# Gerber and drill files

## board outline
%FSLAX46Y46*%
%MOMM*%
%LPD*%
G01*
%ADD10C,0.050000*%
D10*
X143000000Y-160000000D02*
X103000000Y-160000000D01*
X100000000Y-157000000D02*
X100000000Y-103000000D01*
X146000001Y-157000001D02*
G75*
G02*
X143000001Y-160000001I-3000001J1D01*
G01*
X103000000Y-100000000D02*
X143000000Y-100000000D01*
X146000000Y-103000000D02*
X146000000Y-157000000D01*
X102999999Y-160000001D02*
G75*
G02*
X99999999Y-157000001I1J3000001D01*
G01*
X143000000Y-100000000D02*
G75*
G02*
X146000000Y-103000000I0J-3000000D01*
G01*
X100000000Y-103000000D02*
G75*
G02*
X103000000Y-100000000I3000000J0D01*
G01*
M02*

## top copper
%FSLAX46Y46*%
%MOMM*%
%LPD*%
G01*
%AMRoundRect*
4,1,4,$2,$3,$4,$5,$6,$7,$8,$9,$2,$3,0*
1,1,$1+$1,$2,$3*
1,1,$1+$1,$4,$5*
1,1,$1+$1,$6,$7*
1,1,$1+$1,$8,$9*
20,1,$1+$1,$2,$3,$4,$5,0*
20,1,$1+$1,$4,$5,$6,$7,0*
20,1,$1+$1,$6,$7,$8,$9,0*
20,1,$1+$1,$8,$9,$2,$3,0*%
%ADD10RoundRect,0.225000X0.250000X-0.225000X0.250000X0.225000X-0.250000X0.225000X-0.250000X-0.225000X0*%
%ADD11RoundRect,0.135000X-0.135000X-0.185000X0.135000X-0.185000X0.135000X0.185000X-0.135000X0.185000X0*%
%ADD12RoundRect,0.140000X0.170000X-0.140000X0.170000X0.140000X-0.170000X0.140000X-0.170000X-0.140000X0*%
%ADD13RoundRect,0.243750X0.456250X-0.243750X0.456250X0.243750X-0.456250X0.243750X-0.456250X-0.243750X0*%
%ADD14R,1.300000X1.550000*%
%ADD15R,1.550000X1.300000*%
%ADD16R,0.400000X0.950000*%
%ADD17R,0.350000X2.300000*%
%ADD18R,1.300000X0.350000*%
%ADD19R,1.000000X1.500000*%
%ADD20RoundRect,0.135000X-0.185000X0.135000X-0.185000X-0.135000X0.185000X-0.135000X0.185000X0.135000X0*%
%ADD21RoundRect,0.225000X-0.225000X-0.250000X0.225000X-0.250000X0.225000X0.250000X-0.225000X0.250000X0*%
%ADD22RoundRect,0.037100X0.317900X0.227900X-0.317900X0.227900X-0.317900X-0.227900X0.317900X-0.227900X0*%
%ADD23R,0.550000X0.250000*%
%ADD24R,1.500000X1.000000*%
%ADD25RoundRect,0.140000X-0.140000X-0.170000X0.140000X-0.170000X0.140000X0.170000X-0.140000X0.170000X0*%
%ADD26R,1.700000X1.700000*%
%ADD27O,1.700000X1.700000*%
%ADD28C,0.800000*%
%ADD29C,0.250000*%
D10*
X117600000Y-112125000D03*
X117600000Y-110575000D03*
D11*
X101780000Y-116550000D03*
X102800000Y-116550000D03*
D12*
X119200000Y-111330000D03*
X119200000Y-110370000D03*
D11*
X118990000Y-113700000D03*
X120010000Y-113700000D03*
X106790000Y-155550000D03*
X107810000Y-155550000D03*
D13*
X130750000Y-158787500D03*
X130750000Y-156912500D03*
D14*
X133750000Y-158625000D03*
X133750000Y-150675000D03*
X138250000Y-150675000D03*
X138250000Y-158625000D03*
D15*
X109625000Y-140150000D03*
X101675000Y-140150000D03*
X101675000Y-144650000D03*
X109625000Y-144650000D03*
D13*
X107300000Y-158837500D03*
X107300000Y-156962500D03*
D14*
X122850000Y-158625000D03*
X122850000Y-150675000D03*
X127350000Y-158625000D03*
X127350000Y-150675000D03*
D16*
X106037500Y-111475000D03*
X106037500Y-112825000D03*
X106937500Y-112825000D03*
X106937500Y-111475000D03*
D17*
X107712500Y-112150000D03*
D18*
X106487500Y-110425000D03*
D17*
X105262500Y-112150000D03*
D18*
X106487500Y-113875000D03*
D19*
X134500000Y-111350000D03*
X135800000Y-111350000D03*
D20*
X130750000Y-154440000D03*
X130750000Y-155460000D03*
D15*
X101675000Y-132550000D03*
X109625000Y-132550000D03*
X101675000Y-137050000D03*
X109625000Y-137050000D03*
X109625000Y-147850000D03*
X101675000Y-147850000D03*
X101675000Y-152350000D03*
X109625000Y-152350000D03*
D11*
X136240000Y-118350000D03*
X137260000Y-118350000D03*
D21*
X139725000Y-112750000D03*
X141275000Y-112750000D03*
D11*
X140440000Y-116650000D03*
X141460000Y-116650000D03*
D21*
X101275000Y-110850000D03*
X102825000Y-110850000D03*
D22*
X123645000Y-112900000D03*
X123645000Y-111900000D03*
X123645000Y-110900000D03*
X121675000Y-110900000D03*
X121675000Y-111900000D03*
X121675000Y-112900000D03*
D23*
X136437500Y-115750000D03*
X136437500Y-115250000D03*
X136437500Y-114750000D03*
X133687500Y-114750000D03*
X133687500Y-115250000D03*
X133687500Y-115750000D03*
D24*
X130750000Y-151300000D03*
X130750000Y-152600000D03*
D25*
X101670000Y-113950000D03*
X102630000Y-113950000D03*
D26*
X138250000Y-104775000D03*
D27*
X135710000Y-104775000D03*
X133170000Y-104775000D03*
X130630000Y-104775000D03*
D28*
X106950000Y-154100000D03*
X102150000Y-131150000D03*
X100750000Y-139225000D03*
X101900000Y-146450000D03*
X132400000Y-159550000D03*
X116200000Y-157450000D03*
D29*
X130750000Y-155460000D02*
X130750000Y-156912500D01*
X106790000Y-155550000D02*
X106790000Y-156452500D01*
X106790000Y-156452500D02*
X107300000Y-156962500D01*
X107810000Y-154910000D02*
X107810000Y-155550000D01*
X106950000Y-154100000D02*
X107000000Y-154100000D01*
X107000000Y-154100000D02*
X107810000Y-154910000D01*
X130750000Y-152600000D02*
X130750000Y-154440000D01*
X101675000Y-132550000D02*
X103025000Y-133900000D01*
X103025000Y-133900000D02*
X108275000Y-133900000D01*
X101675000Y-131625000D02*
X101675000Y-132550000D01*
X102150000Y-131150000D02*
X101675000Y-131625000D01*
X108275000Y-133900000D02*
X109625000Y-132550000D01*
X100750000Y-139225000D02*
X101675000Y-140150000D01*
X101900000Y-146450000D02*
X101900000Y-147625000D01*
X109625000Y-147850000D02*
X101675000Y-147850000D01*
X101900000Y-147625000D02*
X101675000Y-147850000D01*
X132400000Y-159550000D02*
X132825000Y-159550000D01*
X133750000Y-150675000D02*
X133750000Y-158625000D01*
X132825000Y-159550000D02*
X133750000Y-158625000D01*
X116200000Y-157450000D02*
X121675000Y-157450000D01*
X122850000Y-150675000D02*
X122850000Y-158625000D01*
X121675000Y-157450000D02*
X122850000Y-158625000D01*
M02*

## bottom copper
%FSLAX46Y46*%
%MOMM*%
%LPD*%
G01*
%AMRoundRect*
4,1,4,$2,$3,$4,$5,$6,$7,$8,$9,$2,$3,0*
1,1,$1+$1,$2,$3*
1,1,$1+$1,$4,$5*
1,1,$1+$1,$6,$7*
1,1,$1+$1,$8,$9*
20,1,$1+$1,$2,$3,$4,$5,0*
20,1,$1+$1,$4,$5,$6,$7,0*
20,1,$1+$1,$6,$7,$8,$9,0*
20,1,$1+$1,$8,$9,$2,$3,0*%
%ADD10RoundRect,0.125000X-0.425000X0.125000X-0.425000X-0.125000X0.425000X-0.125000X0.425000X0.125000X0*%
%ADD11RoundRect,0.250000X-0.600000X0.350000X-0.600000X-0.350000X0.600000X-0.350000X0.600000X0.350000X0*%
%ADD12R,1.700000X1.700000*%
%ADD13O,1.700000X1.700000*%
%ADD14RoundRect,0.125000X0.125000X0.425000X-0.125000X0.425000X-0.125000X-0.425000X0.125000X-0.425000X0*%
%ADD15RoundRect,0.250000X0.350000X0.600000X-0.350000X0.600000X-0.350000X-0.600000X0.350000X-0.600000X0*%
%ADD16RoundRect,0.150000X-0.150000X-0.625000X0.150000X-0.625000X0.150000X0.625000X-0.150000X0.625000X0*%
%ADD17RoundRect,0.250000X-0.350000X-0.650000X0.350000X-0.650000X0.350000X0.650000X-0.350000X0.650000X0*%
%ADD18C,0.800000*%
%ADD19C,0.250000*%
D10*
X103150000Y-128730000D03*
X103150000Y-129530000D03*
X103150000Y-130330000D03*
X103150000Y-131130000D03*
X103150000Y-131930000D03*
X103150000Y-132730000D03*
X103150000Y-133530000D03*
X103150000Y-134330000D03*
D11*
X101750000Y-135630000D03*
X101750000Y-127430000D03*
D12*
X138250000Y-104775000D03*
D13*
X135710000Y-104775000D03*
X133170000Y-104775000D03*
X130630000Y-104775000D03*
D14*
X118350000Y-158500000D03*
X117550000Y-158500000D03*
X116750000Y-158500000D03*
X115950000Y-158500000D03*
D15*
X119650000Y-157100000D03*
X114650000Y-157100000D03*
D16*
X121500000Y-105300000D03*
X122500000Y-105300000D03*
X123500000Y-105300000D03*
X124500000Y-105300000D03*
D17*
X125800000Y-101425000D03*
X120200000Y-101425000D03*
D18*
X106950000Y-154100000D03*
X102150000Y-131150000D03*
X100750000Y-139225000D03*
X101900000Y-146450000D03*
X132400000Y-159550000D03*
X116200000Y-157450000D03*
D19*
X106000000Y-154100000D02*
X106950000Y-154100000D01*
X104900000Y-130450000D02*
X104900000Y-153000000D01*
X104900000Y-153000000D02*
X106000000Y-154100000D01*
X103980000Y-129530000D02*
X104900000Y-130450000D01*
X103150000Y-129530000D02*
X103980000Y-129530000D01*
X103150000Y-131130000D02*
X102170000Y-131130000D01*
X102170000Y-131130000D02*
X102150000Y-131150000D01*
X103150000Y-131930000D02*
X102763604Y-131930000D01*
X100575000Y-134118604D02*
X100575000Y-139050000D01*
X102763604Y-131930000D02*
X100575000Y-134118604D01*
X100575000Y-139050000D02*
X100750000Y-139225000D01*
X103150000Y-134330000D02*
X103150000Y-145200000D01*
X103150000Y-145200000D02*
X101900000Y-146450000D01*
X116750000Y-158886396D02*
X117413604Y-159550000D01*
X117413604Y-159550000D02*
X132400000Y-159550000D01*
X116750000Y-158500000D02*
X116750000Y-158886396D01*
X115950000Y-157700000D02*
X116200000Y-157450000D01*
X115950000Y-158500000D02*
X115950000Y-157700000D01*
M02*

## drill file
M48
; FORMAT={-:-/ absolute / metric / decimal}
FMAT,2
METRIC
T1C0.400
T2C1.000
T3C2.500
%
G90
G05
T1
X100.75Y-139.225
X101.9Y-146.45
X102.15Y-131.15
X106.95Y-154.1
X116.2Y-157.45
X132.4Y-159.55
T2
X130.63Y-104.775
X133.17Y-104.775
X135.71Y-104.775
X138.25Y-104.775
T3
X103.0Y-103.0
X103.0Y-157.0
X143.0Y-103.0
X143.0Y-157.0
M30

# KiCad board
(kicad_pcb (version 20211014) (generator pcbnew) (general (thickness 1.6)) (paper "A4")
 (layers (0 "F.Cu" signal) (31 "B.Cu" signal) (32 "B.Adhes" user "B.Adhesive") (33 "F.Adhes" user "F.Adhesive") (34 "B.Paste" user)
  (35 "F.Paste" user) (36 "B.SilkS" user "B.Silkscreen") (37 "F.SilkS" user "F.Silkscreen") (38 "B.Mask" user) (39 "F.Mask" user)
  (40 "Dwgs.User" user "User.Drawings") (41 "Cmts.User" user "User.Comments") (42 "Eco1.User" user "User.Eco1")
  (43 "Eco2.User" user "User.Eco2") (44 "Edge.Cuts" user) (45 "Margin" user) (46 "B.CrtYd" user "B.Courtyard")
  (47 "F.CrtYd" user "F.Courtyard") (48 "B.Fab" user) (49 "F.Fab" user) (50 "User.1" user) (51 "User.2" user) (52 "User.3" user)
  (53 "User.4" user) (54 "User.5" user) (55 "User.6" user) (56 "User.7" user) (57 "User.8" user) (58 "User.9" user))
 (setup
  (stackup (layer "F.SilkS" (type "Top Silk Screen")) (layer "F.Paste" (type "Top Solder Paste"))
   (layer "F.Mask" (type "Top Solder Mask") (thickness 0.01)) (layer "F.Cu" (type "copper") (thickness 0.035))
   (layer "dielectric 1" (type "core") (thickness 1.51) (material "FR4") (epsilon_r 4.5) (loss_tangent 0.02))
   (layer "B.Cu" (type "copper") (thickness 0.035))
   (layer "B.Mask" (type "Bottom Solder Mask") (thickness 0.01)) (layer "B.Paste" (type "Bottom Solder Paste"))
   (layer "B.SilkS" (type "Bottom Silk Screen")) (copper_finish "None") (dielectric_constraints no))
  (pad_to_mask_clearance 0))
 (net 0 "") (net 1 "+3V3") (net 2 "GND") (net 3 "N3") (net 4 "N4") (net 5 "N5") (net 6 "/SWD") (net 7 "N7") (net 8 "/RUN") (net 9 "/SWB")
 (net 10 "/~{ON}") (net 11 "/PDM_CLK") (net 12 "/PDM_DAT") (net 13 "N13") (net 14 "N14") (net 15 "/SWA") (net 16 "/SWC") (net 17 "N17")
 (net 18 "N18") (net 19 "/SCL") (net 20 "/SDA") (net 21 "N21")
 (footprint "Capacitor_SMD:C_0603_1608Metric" (layer "F.Cu") (at 117.6 111.35 90)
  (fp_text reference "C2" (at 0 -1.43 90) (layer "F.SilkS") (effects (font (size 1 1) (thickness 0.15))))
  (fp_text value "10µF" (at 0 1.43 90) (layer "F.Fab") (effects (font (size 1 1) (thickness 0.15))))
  (pad "1" smd roundrect (at -0.775 0 90) (size 0.9 0.95) (layers "F.Cu" "F.Paste" "F.Mask") (roundrect_rratio 0.25) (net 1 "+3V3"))
  (pad "2" smd roundrect (at 0.775 0 90) (size 0.9 0.95) (layers "F.Cu" "F.Paste" "F.Mask") (roundrect_rratio 0.25) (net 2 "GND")))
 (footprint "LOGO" (layer "F.Cu") (at 123.25 129.55)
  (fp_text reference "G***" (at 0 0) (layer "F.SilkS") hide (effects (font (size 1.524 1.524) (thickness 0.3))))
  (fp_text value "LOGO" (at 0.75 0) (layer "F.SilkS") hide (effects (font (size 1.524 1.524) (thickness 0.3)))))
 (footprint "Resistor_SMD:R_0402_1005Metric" (layer "F.Cu") (at 102.29 116.55)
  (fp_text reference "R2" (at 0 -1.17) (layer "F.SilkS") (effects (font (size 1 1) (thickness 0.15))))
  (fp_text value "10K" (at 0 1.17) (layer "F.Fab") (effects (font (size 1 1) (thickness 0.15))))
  (pad "1" smd roundrect (at -0.51 0) (size 0.54 0.64) (layers "F.Cu" "F.Paste" "F.Mask") (roundrect_rratio 0.25) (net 2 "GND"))
  (pad "2" smd roundrect (at 0.51 0) (size 0.54 0.64) (layers "F.Cu" "F.Paste" "F.Mask") (roundrect_rratio 0.25) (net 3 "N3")))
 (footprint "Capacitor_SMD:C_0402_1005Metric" (layer "F.Cu") (at 119.2 110.85 90)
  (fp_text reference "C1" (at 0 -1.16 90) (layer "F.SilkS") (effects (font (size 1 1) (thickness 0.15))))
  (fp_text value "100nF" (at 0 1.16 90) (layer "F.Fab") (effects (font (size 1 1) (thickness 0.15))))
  (pad "1" smd roundrect (at -0.48 0 90) (size 0.56 0.62) (layers "F.Cu" "F.Paste" "F.Mask") (roundrect_rratio 0.25) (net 1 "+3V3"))
  (pad "2" smd roundrect (at 0.48 0 90) (size 0.56 0.62) (layers "F.Cu" "F.Paste" "F.Mask") (roundrect_rratio 0.25) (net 2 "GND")))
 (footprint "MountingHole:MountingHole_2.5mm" (layer "F.Cu") (at 103 103)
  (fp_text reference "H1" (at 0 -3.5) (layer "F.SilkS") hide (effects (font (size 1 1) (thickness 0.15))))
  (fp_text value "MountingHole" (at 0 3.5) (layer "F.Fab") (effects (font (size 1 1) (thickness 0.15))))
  (pad "" np_thru_hole circle (at 0 0) (size 2.5 2.5) (drill 2.5) (layers *.Cu *.Mask)))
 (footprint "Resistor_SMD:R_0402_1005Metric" (layer "F.Cu") (at 119.5 113.7)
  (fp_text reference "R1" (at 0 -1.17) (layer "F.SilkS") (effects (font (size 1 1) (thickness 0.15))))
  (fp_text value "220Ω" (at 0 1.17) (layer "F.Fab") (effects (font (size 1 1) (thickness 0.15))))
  (pad "1" smd roundrect (at -0.51 0) (size 0.54 0.64) (layers "F.Cu" "F.Paste" "F.Mask") (roundrect_rratio 0.25) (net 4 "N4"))
  (pad "2" smd roundrect (at 0.51 0) (size 0.54 0.64) (layers "F.Cu" "F.Paste" "F.Mask") (roundrect_rratio 0.25) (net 1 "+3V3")))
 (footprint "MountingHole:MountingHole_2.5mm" (layer "F.Cu") (at 143 103)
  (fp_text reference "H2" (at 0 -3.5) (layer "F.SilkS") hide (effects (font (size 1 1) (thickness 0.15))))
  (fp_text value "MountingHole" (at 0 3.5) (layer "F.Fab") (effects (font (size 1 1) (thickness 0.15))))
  (pad "" np_thru_hole circle (at 0 0) (size 2.5 2.5) (drill 2.5) (layers *.Cu *.Mask)))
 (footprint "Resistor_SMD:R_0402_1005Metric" (layer "F.Cu") (at 107.3 155.55)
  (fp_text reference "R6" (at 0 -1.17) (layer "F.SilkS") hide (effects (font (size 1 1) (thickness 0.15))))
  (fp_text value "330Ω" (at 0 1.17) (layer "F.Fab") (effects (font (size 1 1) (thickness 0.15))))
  (pad "1" smd roundrect (at -0.51 0) (size 0.54 0.64) (layers "F.Cu" "F.Paste" "F.Mask") (roundrect_rratio 0.25) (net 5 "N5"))
  (pad "2" smd roundrect (at 0.51 0) (size 0.54 0.64) (layers "F.Cu" "F.Paste" "F.Mask") (roundrect_rratio 0.25) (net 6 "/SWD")))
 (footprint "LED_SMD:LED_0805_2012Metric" (layer "F.Cu") (at 130.75 157.85 90)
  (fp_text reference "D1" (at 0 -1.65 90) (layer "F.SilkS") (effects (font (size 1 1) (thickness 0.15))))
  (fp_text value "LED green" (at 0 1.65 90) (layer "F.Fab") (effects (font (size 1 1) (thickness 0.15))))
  (pad "1" smd roundrect (at -0.9375 0 90) (size 0.975 1.4) (layers "F.Cu" "F.Paste" "F.Mask") (roundrect_rratio 0.25) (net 2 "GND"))
  (pad "2" smd roundrect (at 0.9375 0 90) (size 0.975 1.4) (layers "F.Cu" "F.Paste" "F.Mask") (roundrect_rratio 0.25) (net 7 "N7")))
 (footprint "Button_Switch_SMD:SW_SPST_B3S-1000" (layer "F.Cu") (at 136 154.65 90)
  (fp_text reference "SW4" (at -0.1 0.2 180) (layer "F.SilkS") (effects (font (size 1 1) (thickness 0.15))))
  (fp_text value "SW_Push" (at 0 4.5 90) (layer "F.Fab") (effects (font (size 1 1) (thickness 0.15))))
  (pad "1" smd rect (at -3.975 -2.25 90) (size 1.55 1.3) (layers "F.Cu" "F.Paste" "F.Mask") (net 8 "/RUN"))
  (pad "1" smd rect (at 3.975 -2.25 90) (size 1.55 1.3) (layers "F.Cu" "F.Paste" "F.Mask") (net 8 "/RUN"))
  (pad "2" smd rect (at 3.975 2.25 90) (size 1.55 1.3) (layers "F.Cu" "F.Paste" "F.Mask") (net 2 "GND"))
  (pad "2" smd rect (at -3.975 2.25 90) (size 1.55 1.3) (layers "F.Cu" "F.Paste" "F.Mask") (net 2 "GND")))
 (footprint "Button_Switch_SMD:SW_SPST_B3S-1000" (layer "F.Cu") (at 105.65 142.4)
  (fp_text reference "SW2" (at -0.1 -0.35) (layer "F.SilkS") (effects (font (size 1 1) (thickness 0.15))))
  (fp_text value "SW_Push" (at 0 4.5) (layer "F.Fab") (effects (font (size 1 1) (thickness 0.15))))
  (pad "1" smd rect (at 3.975 -2.25) (size 1.55 1.3) (layers "F.Cu" "F.Paste" "F.Mask") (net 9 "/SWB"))
  (pad "1" smd rect (at -3.975 -2.25) (size 1.55 1.3) (layers "F.Cu" "F.Paste" "F.Mask") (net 9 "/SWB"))
  (pad "2" smd rect (at -3.975 2.25) (size 1.55 1.3) (layers "F.Cu" "F.Paste" "F.Mask") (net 2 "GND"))
  (pad "2" smd rect (at 3.975 2.25) (size 1.55 1.3) (layers "F.Cu" "F.Paste" "F.Mask") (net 2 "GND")))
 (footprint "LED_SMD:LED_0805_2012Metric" (layer "F.Cu") (at 107.3 157.9 90)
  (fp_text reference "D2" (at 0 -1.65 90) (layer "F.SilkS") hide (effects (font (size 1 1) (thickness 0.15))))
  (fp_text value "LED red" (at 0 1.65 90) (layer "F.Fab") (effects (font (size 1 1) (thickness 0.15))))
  (pad "1" smd roundrect (at -0.9375 0 90) (size 0.975 1.4) (layers "F.Cu" "F.Paste" "F.Mask") (roundrect_rratio 0.25) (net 2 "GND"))
  (pad "2" smd roundrect (at 0.9375 0 90) (size 0.975 1.4) (layers "F.Cu" "F.Paste" "F.Mask") (roundrect_rratio 0.25) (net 5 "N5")))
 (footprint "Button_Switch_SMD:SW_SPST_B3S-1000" (layer "F.Cu") (at 125.1 154.65 90)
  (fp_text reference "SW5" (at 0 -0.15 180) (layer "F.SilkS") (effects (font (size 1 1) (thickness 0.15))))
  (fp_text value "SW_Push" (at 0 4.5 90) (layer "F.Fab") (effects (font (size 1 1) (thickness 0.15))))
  (pad "1" smd rect (at -3.975 -2.25 90) (size 1.55 1.3) (layers "F.Cu" "F.Paste" "F.Mask") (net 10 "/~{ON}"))
  (pad "1" smd rect (at 3.975 -2.25 90) (size 1.55 1.3) (layers "F.Cu" "F.Paste" "F.Mask") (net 10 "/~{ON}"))
  (pad "2" smd rect (at -3.975 2.25 90) (size 1.55 1.3) (layers "F.Cu" "F.Paste" "F.Mask") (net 2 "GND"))
  (pad "2" smd rect (at 3.975 2.25 90) (size 1.55 1.3) (layers "F.Cu" "F.Paste" "F.Mask") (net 2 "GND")))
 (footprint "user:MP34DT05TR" (layer "F.Cu") (at 106.4875 112.15)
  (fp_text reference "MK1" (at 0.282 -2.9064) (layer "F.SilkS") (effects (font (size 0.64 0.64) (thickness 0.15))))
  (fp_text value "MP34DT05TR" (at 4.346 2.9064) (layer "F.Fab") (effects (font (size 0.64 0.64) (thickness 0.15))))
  (pad "1" smd rect locked (at -0.45 -0.675 180) (size 0.4 0.95) (layers "F.Cu" "F.Paste" "F.Mask") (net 1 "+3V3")
   (solder_mask_margin 0.102))
  (pad "2" smd rect locked (at -0.45 0.675 180) (size 0.4 0.95) (layers "F.Cu" "F.Paste" "F.Mask") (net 3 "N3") (solder_mask_margin 0.102))
  (pad "3" smd rect locked (at 0.45 0.675 180) (size 0.4 0.95) (layers "F.Cu" "F.Paste" "F.Mask") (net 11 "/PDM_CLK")
   (solder_mask_margin 0.102))
  (pad "4" smd rect locked (at 0.45 -0.675 180) (size 0.4 0.95) (layers "F.Cu" "F.Paste" "F.Mask") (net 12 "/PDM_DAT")
   (solder_mask_margin 0.102))
  (pad "5" smd rect locked (at 1.225 0 180) (size 0.35 2.3) (layers "F.Cu" "F.Paste" "F.Mask") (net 2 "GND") (solder_mask_margin 0.102))
  (pad "6" smd rect locked (at 0 -1.725 180) (size 1.3 0.35) (layers "F.Cu" "F.Paste" "F.Mask") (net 2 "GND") (solder_mask_margin 0.102))
  (pad "7" smd rect locked (at -1.225 0 180) (size 0.35 2.3) (layers "F.Cu" "F.Paste" "F.Mask") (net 2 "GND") (solder_mask_margin 0.102))
  (pad "8" smd rect locked (at 0 1.725 180) (size 1.3 0.35) (layers "F.Cu" "F.Paste" "F.Mask") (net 2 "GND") (solder_mask_margin 0.102)))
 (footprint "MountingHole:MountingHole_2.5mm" (layer "F.Cu") (at 143 157)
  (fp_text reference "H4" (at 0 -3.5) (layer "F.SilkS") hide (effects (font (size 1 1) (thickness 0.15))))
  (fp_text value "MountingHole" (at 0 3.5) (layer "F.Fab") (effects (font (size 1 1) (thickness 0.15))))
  (pad "" np_thru_hole circle (at 0 0) (size 2.5 2.5) (drill 2.5) (layers *.Cu *.Mask)))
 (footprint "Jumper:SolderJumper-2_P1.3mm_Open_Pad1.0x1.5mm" (layer "F.Cu") (at 135.15 111.35)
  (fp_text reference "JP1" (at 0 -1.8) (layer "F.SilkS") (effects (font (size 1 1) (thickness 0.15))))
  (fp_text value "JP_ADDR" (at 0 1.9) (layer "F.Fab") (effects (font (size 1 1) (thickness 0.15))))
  (pad "1" smd rect (at -0.65 0) (size 1 1.5) (layers "F.Cu" "F.Mask") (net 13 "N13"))
  (pad "2" smd rect (at 0.65 0) (size 1 1.5) (layers "F.Cu" "F.Mask") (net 1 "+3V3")))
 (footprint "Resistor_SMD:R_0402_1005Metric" (layer "F.Cu") (at 130.75 154.95 -90)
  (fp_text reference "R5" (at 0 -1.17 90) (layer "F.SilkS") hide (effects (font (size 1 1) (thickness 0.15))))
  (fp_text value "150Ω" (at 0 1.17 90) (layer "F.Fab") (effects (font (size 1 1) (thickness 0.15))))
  (pad "1" smd roundrect (at -0.51 0 270) (size 0.54 0.64) (layers "F.Cu" "F.Paste" "F.Mask") (roundrect_rratio 0.25) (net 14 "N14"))
  (pad "2" smd roundrect (at 0.51 0 270) (size 0.54 0.64) (layers "F.Cu" "F.Paste" "F.Mask") (roundrect_rratio 0.25) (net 7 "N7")))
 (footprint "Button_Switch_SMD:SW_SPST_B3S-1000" (layer "F.Cu") (at 105.65 134.8)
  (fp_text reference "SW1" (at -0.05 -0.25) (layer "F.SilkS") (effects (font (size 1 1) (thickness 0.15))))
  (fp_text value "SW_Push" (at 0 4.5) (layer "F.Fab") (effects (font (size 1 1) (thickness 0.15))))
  (pad "1" smd rect (at -3.975 -2.25) (size 1.55 1.3) (layers "F.Cu" "F.Paste" "F.Mask") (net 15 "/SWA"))
  (pad "1" smd rect (at 3.975 -2.25) (size 1.55 1.3) (layers "F.Cu" "F.Paste" "F.Mask") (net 15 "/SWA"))
  (pad "2" smd rect (at -3.975 2.25) (size 1.55 1.3) (layers "F.Cu" "F.Paste" "F.Mask") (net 2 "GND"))
  (pad "2" smd rect (at 3.975 2.25) (size 1.55 1.3) (layers "F.Cu" "F.Paste" "F.Mask") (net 2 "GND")))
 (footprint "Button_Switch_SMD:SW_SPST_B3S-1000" (layer "F.Cu") (at 105.65 150.1)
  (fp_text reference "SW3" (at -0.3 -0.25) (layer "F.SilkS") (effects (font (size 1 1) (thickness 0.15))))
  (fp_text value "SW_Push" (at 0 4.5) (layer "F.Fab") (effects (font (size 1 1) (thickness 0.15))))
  (pad "1" smd rect (at 3.975 -2.25) (size 1.55 1.3) (layers "F.Cu" "F.Paste" "F.Mask") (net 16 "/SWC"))
  (pad "1" smd rect (at -3.975 -2.25) (size 1.55 1.3) (layers "F.Cu" "F.Paste" "F.Mask") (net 16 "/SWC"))
  (pad "2" smd rect (at -3.975 2.25) (size 1.55 1.3) (layers "F.Cu" "F.Paste" "F.Mask") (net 2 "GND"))
  (pad "2" smd rect (at 3.975 2.25) (size 1.55 1.3) (layers "F.Cu" "F.Paste" "F.Mask") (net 2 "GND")))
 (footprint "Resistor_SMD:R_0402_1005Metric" (layer "F.Cu") (at 136.75 118.35)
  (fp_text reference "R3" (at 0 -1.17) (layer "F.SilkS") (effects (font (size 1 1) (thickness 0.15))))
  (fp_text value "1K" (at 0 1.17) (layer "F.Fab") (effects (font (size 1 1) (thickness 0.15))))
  (pad "1" smd roundrect (at -0.51 0) (size 0.54 0.64) (layers "F.Cu" "F.Paste" "F.Mask") (roundrect_rratio 0.25) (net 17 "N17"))
  (pad "2" smd roundrect (at 0.51 0) (size 0.54 0.64) (layers "F.Cu" "F.Paste" "F.Mask") (roundrect_rratio 0.25) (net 1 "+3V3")))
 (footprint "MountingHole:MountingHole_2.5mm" (layer "F.Cu") (at 103 157)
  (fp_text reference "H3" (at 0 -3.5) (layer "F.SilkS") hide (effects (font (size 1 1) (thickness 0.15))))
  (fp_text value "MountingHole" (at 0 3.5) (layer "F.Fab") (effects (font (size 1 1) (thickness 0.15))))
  (pad "" np_thru_hole circle (at 0 0) (size 2.5 2.5) (drill 2.5) (layers *.Cu *.Mask)))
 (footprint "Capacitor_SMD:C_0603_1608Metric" (layer "F.Cu") (at 140.5 112.75)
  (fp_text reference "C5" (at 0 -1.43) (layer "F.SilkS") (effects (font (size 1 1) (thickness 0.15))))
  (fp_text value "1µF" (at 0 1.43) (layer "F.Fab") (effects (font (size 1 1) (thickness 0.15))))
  (pad "1" smd roundrect (at -0.775 0) (size 0.9 0.95) (layers "F.Cu" "F.Paste" "F.Mask") (roundrect_rratio 0.25) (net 2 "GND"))
  (pad "2" smd roundrect (at 0.775 0) (size 0.9 0.95) (layers "F.Cu" "F.Paste" "F.Mask") (roundrect_rratio 0.25) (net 17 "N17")))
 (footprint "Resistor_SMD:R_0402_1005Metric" (layer "F.Cu") (at 140.95 116.65)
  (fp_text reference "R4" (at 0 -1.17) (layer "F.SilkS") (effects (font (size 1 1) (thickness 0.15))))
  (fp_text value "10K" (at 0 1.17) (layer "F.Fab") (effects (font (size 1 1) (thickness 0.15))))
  (pad "1" smd roundrect (at -0.51 0) (size 0.54 0.64) (layers "F.Cu" "F.Paste" "F.Mask") (roundrect_rratio 0.25) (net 13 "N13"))
  (pad "2" smd roundrect (at 0.51 0) (size 0.54 0.64) (layers "F.Cu" "F.Paste" "F.Mask") (roundrect_rratio 0.25) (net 2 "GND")))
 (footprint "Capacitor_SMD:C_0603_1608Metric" (layer "F.Cu") (at 102.05 110.85)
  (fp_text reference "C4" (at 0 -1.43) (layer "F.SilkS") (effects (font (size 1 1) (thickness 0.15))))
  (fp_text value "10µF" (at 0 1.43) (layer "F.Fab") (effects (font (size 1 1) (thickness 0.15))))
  (pad "1" smd roundrect (at -0.775 0) (size 0.9 0.95) (layers "F.Cu" "F.Paste" "F.Mask") (roundrect_rratio 0.25) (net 1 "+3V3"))
  (pad "2" smd roundrect (at 0.775 0) (size 0.9 0.95) (layers "F.Cu" "F.Paste" "F.Mask") (roundrect_rratio 0.25) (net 2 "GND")))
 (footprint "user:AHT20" (layer "F.Cu") (at 122.66 111.9 180)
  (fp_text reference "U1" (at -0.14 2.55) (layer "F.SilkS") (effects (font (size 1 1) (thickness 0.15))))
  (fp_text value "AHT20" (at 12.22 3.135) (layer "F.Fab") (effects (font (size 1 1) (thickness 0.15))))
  (pad "1" smd roundrect locked (at -0.985 -1 180) (size 0.71 0.53) (layers "F.Cu" "F.Paste" "F.Mask") (roundrect_rratio 0.07)
   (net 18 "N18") (solder_mask_margin 0.102))
  (pad "2" smd roundrect locked (at -0.985 0 180) (size 0.71 0.53) (layers "F.Cu" "F.Paste" "F.Mask") (roundrect_rratio 0.07) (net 4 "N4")
   (solder_mask_margin 0.102))
  (pad "3" smd roundrect locked (at -0.985 1 180) (size 0.71 0.53) (layers "F.Cu" "F.Paste" "F.Mask") (roundrect_rratio 0.07)
   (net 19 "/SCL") (solder_mask_margin 0.102))
  (pad "4" smd roundrect locked (at 0.985 1 180) (size 0.71 0.53) (layers "F.Cu" "F.Paste" "F.Mask") (roundrect_rratio 0.07) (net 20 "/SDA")
   (solder_mask_margin 0.102))
  (pad "5" smd roundrect locked (at 0.985 0 180) (size 0.71 0.53) (layers "F.Cu" "F.Paste" "F.Mask") (roundrect_rratio 0.07) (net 2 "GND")
   (solder_mask_margin 0.102))
  (pad "6" smd roundrect locked (at 0.985 -1 180) (size 0.71 0.53) (layers "F.Cu" "F.Paste" "F.Mask") (roundrect_rratio 0.07) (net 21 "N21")
   (solder_mask_margin 0.102)))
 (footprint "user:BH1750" (layer "F.Cu") (at 135.0625 115.25 180)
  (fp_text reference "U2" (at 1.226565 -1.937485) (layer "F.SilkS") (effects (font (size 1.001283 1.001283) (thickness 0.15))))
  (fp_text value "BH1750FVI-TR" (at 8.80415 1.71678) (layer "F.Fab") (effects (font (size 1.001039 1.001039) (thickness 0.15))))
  (pad "1" smd rect locked (at -1.375 -0.5 180) (size 0.55 0.25) (layers "F.Cu" "F.Paste" "F.Mask") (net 1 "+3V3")
   (solder_mask_margin 0.102))
  (pad "2" smd rect locked (at -1.375 0 180) (size 0.55 0.25) (layers "F.Cu" "F.Paste" "F.Mask") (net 13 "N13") (solder_mask_margin 0.102))
  (pad "3" smd rect locked (at -1.375 0.5 180) (size 0.55 0.25) (layers "F.Cu" "F.Paste" "F.Mask") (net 2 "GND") (solder_mask_margin 0.102))
  (pad "4" smd rect locked (at 1.375 0.5 180) (size 0.55 0.25) (layers "F.Cu" "F.Paste" "F.Mask") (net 20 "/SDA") (solder_mask_margin 0.102))
  (pad "5" smd rect locked (at 1.375 0 180) (size 0.55 0.25) (layers "F.Cu" "F.Paste" "F.Mask") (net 17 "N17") (solder_mask_margin 0.102))
  (pad "6" smd rect locked (at 1.375 -0.5 180) (size 0.55 0.25) (layers "F.Cu" "F.Paste" "F.Mask") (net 19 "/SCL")
   (solder_mask_margin 0.102)))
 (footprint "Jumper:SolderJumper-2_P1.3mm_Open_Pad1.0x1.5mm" (layer "F.Cu") (at 130.75 151.95 -90)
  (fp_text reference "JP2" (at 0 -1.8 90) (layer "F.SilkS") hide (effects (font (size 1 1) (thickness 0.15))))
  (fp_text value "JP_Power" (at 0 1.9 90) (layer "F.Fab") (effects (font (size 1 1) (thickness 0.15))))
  (pad "1" smd rect (at -0.65 0 270) (size 1 1.5) (layers "F.Cu" "F.Mask") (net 1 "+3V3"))
  (pad "2" smd rect (at 0.65 0 270) (size 1 1.5) (layers "F.Cu" "F.Mask") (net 14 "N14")))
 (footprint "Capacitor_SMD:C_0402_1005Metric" (layer "F.Cu") (at 102.15 113.95)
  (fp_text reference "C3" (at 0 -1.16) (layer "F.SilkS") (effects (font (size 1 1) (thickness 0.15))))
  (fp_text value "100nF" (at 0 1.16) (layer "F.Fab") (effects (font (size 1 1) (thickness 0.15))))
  (pad "1" smd roundrect (at -0.48 0) (size 0.56 0.62) (layers "F.Cu" "F.Paste" "F.Mask") (roundrect_rratio 0.25) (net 1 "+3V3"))
  (pad "2" smd roundrect (at 0.48 0) (size 0.56 0.62) (layers "F.Cu" "F.Paste" "F.Mask") (roundrect_rratio 0.25) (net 2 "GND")))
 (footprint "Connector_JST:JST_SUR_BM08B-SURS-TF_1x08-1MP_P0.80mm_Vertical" (layer "B.Cu") (at 102.3 131.53 -90)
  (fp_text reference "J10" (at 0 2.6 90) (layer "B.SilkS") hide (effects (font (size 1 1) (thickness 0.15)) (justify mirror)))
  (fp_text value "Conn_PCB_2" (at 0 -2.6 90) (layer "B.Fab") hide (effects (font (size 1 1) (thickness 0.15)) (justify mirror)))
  (pad "1" smd roundrect (at -2.8 -0.85 270) (size 0.5 1.1) (layers "B.Cu" "B.Paste" "B.Mask") (roundrect_rratio 0.25) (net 11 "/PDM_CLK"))
  (pad "2" smd roundrect (at -2 -0.85 270) (size 0.5 1.1) (layers "B.Cu" "B.Paste" "B.Mask") (roundrect_rratio 0.25) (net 6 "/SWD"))
  (pad "3" smd roundrect (at -1.2 -0.85 270) (size 0.5 1.1) (layers "B.Cu" "B.Paste" "B.Mask") (roundrect_rratio 0.25) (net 12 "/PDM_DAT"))
  (pad "4" smd roundrect (at -0.4 -0.85 270) (size 0.5 1.1) (layers "B.Cu" "B.Paste" "B.Mask") (roundrect_rratio 0.25) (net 15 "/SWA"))
  (pad "5" smd roundrect (at 0.4 -0.85 270) (size 0.5 1.1) (layers "B.Cu" "B.Paste" "B.Mask") (roundrect_rratio 0.25) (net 9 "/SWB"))
  (pad "6" smd roundrect (at 1.2 -0.85 270) (size 0.5 1.1) (layers "B.Cu" "B.Paste" "B.Mask") (roundrect_rratio 0.25) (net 20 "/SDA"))
  (pad "7" smd roundrect (at 2 -0.85 270) (size 0.5 1.1) (layers "B.Cu" "B.Paste" "B.Mask") (roundrect_rratio 0.25) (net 19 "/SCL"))
  (pad "8" smd roundrect (at 2.8 -0.85 270) (size 0.5 1.1) (layers "B.Cu" "B.Paste" "B.Mask") (roundrect_rratio 0.25) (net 16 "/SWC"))
  (pad "MP" smd roundrect (at 4.1 0.55 270) (size 1.2 1.7) (layers "B.Cu" "B.Paste" "B.Mask") (roundrect_rratio 0.2083333333))
  (pad "MP" smd roundrect (at -4.1 0.55 270) (size 1.2 1.7) (layers "B.Cu" "B.Paste" "B.Mask") (roundrect_rratio 0.2083333333)))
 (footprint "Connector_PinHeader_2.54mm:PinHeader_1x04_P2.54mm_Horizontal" (layer "B.Cu") (at 138.25 104.775 90)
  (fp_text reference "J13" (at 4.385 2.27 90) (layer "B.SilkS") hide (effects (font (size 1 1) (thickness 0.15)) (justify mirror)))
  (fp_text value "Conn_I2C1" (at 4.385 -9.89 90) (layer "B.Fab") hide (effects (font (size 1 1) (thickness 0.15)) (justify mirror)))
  (pad "1" thru_hole rect (at 0 0 90) (size 1.7 1.7) (drill 1) (layers *.Cu *.Mask) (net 2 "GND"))
  (pad "2" thru_hole oval (at 0 -2.54 90) (size 1.7 1.7) (drill 1) (layers *.Cu *.Mask) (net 1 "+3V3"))
  (pad "3" thru_hole oval (at 0 -5.08 90) (size 1.7 1.7) (drill 1) (layers *.Cu *.Mask) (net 20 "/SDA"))
  (pad "4" thru_hole oval (at 0 -7.62 90) (size 1.7 1.7) (drill 1) (layers *.Cu *.Mask) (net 19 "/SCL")))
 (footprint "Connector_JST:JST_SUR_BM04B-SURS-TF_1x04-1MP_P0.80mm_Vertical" (layer "B.Cu") (at 117.15 157.65 180)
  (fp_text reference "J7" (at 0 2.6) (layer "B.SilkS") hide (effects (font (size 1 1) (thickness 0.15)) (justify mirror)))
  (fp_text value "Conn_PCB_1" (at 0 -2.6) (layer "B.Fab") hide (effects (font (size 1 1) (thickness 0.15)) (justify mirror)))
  (pad "1" smd roundrect (at -1.2 -0.85 180) (size 0.5 1.1) (layers "B.Cu" "B.Paste" "B.Mask") (roundrect_rratio 0.25) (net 2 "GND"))
  (pad "2" smd roundrect (at -0.4 -0.85 180) (size 0.5 1.1) (layers "B.Cu" "B.Paste" "B.Mask") (roundrect_rratio 0.25) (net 1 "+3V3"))
  (pad "3" smd roundrect (at 0.4 -0.85 180) (size 0.5 1.1) (layers "B.Cu" "B.Paste" "B.Mask") (roundrect_rratio 0.25) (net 8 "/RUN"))
  (pad "4" smd roundrect (at 1.2 -0.85 180) (size 0.5 1.1) (layers "B.Cu" "B.Paste" "B.Mask") (roundrect_rratio 0.25) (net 10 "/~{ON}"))
  (pad "MP" smd roundrect (at -2.5 0.55 180) (size 1.2 1.7) (layers "B.Cu" "B.Paste" "B.Mask") (roundrect_rratio 0.2083333333))
  (pad "MP" smd roundrect (at 2.5 0.55 180) (size 1.2 1.7) (layers "B.Cu" "B.Paste" "B.Mask") (roundrect_rratio 0.2083333333)))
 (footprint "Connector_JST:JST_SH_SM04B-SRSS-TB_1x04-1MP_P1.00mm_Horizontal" (layer "B.Cu") (at 123 103.3)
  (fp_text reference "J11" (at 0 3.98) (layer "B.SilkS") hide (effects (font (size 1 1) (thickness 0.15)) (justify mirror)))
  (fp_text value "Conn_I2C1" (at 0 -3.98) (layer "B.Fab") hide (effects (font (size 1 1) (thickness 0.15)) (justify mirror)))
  (pad "1" smd roundrect (at -1.5 2) (size 0.6 1.55) (layers "B.Cu" "B.Paste" "B.Mask") (roundrect_rratio 0.25) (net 2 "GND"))
  (pad "2" smd roundrect (at -0.5 2) (size 0.6 1.55) (layers "B.Cu" "B.Paste" "B.Mask") (roundrect_rratio 0.25) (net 1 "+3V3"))
  (pad "3" smd roundrect (at 0.5 2) (size 0.6 1.55) (layers "B.Cu" "B.Paste" "B.Mask") (roundrect_rratio 0.25) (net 20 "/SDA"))
  (pad "4" smd roundrect (at 1.5 2) (size 0.6 1.55) (layers "B.Cu" "B.Paste" "B.Mask") (roundrect_rratio 0.25) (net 19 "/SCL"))
  (pad "MP" smd roundrect (at 2.8 -1.875) (size 1.2 1.8) (layers "B.Cu" "B.Paste" "B.Mask") (roundrect_rratio 0.208333))
  (pad "MP" smd roundrect (at -2.8 -1.875) (size 1.2 1.8) (layers "B.Cu" "B.Paste" "B.Mask") (roundrect_rratio 0.208333)))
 (gr_line (start 143 160) (end 103 160) (layer "Edge.Cuts") (width 0.05))
 (gr_line (start 100 157) (end 100 103) (layer "Edge.Cuts") (width 0.05))
 (gr_arc (start 146.000001 157.000001) (mid 145.121321 159.121321) (end 143.000001 160.000001) (layer "Edge.Cuts") (width 0.05))
 (gr_line (start 103 100) (end 143 100) (layer "Edge.Cuts") (width 0.05))
 (gr_line (start 146 103) (end 146 157) (layer "Edge.Cuts") (width 0.05))
 (gr_arc (start 102.999999 160.000001) (mid 100.878679 159.121321) (end 99.999999 157.000001) (layer "Edge.Cuts") (width 0.05))
 (gr_arc (start 143 100) (mid 145.12132 100.87868) (end 146 103) (layer "Edge.Cuts") (width 0.05))
 (gr_arc (start 100 103) (mid 100.87868 100.87868) (end 103 100) (layer "Edge.Cuts") (width 0.05))
 (segment (start 130.75 155.46) (end 130.75 156.9125) (width 0.25) (layer "F.Cu") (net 7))
 (segment (start 106.79 155.55) (end 106.79 156.4525) (width 0.25) (layer "F.Cu") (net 5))
 (segment (start 106.79 156.4525) (end 107.3 156.9625) (width 0.25) (layer "F.Cu") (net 5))
 (segment (start 107.81 154.91) (end 107.81 155.55) (width 0.25) (layer "F.Cu") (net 6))
 (segment (start 106.95 154.1) (end 107 154.1) (width 0.25) (layer "F.Cu") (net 6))
 (segment (start 107 154.1) (end 107.81 154.91) (width 0.25) (layer "F.Cu") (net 6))
 (via (at 106.95 154.1) (size 0.8) (drill 0.4) (layers "F.Cu" "B.Cu") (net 6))
 (segment (start 106 154.1) (end 106.95 154.1) (width 0.25) (layer "B.Cu") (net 6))
 (segment (start 104.9 130.45) (end 104.9 153) (width 0.25) (layer "B.Cu") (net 6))
 (segment (start 104.9 153) (end 106 154.1) (width 0.25) (layer "B.Cu") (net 6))
 (segment (start 103.98 129.53) (end 104.9 130.45) (width 0.25) (layer "B.Cu") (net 6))
 (segment (start 103.15 129.53) (end 103.98 129.53) (width 0.25) (layer "B.Cu") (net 6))
 (segment (start 130.75 152.6) (end 130.75 154.44) (width 0.25) (layer "F.Cu") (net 14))
 (segment (start 101.675 132.55) (end 103.025 133.9) (width 0.25) (layer "F.Cu") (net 15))
 (segment (start 103.025 133.9) (end 108.275 133.9) (width 0.25) (layer "F.Cu") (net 15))
 (segment (start 101.675 131.625) (end 101.675 132.55) (width 0.25) (layer "F.Cu") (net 15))
 (segment (start 102.15 131.15) (end 101.675 131.625) (width 0.25) (layer "F.Cu") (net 15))
 (segment (start 108.275 133.9) (end 109.625 132.55) (width 0.25) (layer "F.Cu") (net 15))
 (via (at 102.15 131.15) (size 0.8) (drill 0.4) (layers "F.Cu" "B.Cu") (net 15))
 (segment (start 103.15 131.13) (end 102.17 131.13) (width 0.25) (layer "B.Cu") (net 15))
 (segment (start 102.17 131.13) (end 102.15 131.15) (width 0.25) (layer "B.Cu") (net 15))
 (segment (start 100.75 139.225) (end 101.675 140.15) (width 0.25) (layer "F.Cu") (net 9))
 (via (at 100.75 139.225) (size 0.8) (drill 0.4) (layers "F.Cu" "B.Cu") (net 9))
 (segment (start 103.15 131.93) (end 102.763604 131.93) (width 0.25) (layer "B.Cu") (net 9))
 (segment (start 100.575 134.118604) (end 100.575 139.05) (width 0.25) (layer "B.Cu") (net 9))
 (segment (start 102.763604 131.93) (end 100.575 134.118604) (width 0.25) (layer "B.Cu") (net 9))
 (segment (start 100.575 139.05) (end 100.75 139.225) (width 0.25) (layer "B.Cu") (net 9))
 (segment (start 101.9 146.45) (end 101.9 147.625) (width 0.25) (layer "F.Cu") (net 16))
 (segment (start 109.625 147.85) (end 101.675 147.85) (width 0.25) (layer "F.Cu") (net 16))
 (segment (start 101.9 147.625) (end 101.675 147.85) (width 0.25) (layer "F.Cu") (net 16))
 (via (at 101.9 146.45) (size 0.8) (drill 0.4) (layers "F.Cu" "B.Cu") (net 16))
 (segment (start 103.15 134.33) (end 103.15 145.2) (width 0.25) (layer "B.Cu") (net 16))
 (segment (start 103.15 145.2) (end 101.9 146.45) (width 0.25) (layer "B.Cu") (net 16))
 (segment (start 132.4 159.55) (end 132.825 159.55) (width 0.25) (layer "F.Cu") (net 8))
 (segment (start 133.75 150.675) (end 133.75 158.625) (width 0.25) (layer "F.Cu") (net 8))
 (segment (start 132.825 159.55) (end 133.75 158.625) (width 0.25) (layer "F.Cu") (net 8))
 (via (at 132.4 159.55) (size 0.8) (drill 0.4) (layers "F.Cu" "B.Cu") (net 8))
 (segment (start 116.75 158.886396) (end 117.413604 159.55) (width 0.25) (layer "B.Cu") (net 8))
 (segment (start 117.413604 159.55) (end 132.4 159.55) (width 0.25) (layer "B.Cu") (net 8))
 (segment (start 116.75 158.5) (end 116.75 158.886396) (width 0.25) (layer "B.Cu") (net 8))
 (segment (start 116.2 157.45) (end 121.675 157.45) (width 0.25) (layer "F.Cu") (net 10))
 (segment (start 122.85 150.675) (end 122.85 158.625) (width 0.25) (layer "F.Cu") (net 10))
 (segment (start 121.675 157.45) (end 122.85 158.625) (width 0.25) (layer "F.Cu") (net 10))
 (via (at 116.2 157.45) (size 0.8) (drill 0.4) (layers "F.Cu" "B.Cu") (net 10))
 (segment (start 115.95 157.7) (end 116.2 157.45) (width 0.25) (layer "B.Cu") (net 10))
 (segment (start 115.95 158.5) (end 115.95 157.7) (width 0.25) (layer "B.Cu") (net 10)))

